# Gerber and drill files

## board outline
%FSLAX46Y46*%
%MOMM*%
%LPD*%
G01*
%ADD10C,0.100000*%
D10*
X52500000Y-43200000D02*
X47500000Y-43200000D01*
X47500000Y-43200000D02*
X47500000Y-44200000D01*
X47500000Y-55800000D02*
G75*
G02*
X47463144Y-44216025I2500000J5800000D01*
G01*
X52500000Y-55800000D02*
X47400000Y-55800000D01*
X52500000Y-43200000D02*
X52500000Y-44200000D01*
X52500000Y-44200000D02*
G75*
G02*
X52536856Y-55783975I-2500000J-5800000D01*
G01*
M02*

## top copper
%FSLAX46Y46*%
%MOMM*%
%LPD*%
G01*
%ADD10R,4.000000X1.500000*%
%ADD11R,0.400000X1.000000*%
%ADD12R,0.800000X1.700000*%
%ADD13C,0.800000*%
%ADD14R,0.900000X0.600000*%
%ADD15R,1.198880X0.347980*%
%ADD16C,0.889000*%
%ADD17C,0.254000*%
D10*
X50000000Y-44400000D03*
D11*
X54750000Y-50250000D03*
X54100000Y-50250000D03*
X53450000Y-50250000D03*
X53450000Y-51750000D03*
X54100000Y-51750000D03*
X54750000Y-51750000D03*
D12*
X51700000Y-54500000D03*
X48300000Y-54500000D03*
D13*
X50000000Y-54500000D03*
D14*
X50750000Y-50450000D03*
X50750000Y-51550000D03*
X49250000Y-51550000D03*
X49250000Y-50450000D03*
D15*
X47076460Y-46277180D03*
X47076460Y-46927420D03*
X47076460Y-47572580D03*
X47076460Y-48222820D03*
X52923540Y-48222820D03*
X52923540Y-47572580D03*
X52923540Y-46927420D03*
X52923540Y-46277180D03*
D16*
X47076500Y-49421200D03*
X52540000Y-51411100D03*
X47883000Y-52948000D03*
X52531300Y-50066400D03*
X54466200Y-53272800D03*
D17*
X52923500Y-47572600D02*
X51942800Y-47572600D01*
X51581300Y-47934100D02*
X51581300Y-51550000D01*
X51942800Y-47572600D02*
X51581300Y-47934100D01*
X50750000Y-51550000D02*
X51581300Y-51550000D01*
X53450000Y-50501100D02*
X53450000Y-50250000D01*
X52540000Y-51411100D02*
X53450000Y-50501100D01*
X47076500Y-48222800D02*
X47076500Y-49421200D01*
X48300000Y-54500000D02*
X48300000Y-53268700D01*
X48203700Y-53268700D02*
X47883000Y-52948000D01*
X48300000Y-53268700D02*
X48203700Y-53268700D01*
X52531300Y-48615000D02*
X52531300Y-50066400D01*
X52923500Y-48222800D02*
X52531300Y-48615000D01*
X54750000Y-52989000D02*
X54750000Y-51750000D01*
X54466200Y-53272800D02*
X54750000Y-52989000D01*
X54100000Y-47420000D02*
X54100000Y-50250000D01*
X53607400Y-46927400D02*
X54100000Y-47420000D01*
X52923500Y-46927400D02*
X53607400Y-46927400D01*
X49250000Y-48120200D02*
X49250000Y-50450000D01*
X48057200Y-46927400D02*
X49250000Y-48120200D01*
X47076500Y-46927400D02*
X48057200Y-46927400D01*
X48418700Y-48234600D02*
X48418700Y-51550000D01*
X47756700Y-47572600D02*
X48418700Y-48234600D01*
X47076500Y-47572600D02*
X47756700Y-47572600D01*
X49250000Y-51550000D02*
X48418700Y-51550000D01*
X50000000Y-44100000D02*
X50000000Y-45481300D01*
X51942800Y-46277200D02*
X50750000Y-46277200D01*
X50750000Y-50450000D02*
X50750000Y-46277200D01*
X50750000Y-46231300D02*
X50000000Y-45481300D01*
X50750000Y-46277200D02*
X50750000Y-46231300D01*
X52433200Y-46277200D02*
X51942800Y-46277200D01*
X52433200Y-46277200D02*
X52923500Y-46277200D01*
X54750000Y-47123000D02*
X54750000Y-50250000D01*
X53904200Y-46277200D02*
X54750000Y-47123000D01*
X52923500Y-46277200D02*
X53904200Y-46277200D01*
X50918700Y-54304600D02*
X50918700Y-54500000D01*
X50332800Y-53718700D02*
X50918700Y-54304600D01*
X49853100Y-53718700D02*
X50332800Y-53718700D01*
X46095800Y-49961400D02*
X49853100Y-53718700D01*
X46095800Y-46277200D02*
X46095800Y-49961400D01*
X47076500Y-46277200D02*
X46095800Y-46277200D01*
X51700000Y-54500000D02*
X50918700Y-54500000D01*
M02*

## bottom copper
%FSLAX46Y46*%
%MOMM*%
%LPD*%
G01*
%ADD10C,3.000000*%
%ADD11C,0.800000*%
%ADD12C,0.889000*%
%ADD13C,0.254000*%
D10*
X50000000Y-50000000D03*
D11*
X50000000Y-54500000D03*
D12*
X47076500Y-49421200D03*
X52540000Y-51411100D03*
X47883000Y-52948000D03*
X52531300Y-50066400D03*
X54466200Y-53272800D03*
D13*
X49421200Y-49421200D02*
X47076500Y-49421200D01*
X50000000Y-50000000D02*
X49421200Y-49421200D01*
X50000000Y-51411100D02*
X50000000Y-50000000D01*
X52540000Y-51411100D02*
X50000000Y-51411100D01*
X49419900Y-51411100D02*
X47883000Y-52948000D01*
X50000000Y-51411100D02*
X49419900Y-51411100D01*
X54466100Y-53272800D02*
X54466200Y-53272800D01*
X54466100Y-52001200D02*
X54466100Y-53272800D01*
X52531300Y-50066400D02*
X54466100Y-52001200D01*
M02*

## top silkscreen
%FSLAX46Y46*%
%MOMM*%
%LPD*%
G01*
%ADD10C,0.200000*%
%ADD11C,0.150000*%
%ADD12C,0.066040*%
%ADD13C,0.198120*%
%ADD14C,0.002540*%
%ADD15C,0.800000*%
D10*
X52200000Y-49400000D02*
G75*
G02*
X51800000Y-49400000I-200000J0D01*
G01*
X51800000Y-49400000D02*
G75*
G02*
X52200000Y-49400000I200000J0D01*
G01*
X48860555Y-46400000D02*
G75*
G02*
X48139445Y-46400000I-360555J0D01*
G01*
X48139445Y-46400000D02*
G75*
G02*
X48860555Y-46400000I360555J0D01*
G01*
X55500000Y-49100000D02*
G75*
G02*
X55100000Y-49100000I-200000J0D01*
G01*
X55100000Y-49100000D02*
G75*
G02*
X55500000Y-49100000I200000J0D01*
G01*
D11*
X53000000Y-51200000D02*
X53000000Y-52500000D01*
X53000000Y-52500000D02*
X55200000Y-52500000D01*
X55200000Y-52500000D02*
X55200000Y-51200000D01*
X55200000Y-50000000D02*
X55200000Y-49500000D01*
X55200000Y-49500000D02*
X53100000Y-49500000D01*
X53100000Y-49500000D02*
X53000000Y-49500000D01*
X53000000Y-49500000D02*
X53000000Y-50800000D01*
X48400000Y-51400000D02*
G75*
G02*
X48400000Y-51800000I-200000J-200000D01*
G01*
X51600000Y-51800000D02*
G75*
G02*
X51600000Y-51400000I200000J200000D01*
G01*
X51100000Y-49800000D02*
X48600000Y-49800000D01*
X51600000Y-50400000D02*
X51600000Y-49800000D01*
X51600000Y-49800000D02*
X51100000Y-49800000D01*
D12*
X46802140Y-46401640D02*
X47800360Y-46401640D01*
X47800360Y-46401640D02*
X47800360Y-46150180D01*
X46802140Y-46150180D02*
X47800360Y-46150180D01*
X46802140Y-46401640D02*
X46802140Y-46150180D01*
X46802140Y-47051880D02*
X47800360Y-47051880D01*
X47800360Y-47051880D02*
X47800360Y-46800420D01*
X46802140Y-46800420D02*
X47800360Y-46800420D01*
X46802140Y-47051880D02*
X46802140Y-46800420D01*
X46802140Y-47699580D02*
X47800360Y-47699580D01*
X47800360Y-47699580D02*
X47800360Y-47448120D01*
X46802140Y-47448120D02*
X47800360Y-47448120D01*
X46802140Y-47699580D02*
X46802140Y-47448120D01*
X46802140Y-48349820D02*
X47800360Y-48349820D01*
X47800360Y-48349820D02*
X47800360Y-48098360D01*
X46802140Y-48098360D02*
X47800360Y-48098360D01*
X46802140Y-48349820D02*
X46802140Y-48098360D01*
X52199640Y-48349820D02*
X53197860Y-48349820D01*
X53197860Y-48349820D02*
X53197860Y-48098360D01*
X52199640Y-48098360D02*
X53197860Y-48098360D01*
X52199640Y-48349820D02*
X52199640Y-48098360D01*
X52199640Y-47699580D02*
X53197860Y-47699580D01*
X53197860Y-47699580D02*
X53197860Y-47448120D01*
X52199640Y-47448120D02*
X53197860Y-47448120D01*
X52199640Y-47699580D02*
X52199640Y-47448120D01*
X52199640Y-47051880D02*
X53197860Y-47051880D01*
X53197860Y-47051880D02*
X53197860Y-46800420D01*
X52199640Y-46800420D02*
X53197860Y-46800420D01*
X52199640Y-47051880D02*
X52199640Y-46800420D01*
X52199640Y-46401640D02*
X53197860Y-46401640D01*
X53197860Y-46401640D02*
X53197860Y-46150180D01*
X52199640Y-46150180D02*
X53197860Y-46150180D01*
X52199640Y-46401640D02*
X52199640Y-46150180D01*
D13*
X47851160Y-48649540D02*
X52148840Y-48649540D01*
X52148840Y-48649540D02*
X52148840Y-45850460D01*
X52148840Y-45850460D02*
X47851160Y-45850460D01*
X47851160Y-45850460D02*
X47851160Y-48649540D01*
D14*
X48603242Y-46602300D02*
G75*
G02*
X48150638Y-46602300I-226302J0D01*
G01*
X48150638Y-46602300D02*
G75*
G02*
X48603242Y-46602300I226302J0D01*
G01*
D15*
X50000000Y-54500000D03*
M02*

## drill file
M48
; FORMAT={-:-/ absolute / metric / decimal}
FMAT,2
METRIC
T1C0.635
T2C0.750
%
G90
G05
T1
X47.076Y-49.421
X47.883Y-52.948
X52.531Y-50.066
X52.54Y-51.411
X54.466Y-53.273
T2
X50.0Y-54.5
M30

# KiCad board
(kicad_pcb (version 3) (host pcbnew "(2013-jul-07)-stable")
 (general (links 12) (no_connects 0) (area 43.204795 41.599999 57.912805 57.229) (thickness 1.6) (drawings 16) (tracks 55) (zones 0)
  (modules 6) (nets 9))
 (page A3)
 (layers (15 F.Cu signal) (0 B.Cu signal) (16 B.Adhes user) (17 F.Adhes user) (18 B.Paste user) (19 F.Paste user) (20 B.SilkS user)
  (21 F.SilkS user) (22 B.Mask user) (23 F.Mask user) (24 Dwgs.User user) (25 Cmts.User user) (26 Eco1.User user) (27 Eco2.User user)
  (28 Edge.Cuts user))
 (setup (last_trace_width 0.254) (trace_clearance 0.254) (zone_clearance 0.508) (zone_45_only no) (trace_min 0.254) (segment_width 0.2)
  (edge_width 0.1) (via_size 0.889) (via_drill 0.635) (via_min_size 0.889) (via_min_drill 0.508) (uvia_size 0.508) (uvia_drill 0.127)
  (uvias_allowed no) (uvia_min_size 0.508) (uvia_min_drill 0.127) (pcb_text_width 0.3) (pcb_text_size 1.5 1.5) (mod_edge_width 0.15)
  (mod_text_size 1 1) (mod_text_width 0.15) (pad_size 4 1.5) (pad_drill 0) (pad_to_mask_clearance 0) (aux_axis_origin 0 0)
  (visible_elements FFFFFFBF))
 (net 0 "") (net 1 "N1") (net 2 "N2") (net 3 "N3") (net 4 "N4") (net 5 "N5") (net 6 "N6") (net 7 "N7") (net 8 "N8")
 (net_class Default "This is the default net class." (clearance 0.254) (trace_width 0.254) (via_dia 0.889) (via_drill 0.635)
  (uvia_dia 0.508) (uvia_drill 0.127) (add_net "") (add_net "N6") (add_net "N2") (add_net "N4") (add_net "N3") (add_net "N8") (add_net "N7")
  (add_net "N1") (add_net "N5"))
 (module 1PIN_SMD (layer F.Cu) (at 50 44.4)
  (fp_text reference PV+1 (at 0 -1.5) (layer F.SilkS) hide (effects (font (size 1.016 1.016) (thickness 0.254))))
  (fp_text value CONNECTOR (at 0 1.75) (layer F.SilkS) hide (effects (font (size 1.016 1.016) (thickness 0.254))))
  (pad 1 smd rect (at 0 0) (size 4 1.5) (layers F.Cu F.Paste F.Mask) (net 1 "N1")))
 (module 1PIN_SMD (layer B.Cu) (at 50 50)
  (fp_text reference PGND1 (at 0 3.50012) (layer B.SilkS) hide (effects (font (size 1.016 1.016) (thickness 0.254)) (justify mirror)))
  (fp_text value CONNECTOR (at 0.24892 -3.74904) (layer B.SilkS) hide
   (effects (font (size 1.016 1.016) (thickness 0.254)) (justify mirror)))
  (pad 1 smd circle (at 0 0) (size 3 3) (layers B.Cu B.Paste B.Mask) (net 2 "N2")))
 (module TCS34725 (layer F.Cu) (at 54.1 51 90)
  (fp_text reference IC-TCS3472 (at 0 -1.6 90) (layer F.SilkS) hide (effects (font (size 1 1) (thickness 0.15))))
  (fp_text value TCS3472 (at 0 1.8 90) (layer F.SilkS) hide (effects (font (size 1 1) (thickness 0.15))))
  (fp_line (start -0.2 -1.1) (end -1.5 -1.1) (layer F.SilkS) (width 0.15))
  (fp_line (start -1.5 -1.1) (end -1.5 1.1) (layer F.SilkS) (width 0.15))
  (fp_line (start -1.5 1.1) (end -0.2 1.1) (layer F.SilkS) (width 0.15))
  (fp_line (start 1 1.1) (end 1.5 1.1) (layer F.SilkS) (width 0.15))
  (fp_line (start 1.5 1.1) (end 1.5 -1) (layer F.SilkS) (width 0.15))
  (fp_line (start 1.5 -1) (end 1.5 -1.1) (layer F.SilkS) (width 0.15))
  (fp_line (start 1.5 -1.1) (end 0.2 -1.1) (layer F.SilkS) (width 0.15))
  (pad 1 smd rect (at 0.75 0.65 90) (size 1 0.4) (layers F.Cu F.Paste F.Mask) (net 1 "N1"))
  (pad 2 smd rect (at 0.75 0 90) (size 1 0.4) (layers F.Cu F.Paste F.Mask) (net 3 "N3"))
  (pad 3 smd rect (at 0.75 -0.65 90) (size 1 0.4) (layers F.Cu F.Paste F.Mask) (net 2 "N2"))
  (pad 4 smd rect (at -0.75 -0.65 90) (size 1 0.4) (layers F.Cu F.Paste F.Mask))
  (pad 5 smd rect (at -0.75 0 90) (size 1 0.4) (layers F.Cu F.Paste F.Mask))
  (pad 6 smd rect (at -0.75 0.65 90) (size 1 0.4) (layers F.Cu F.Paste F.Mask) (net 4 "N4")))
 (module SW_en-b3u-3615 (layer F.Cu) (at 50 54.5 180)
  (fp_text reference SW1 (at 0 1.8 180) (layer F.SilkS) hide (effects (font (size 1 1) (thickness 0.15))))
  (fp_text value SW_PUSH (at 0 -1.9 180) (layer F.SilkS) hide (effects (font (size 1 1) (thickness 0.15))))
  (pad 1 smd rect (at -1.7 0 180) (size 0.8 1.7) (layers F.Cu F.Paste F.Mask) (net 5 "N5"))
  (pad 2 smd rect (at 1.7 0 180) (size 0.8 1.7) (layers F.Cu F.Paste F.Mask) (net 2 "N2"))
  (pad "" thru_hole circle (at 0 0 180) (size 0.8 0.8) (drill 0.75) (layers *.Cu *.Mask F.SilkS)))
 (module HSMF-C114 (layer F.Cu) (at 50 51 180)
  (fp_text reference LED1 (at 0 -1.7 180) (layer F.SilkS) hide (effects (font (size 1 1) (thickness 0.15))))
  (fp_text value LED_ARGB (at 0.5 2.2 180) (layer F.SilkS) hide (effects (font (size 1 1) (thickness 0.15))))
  (fp_arc (start 1.8 -0.6) (end 1.6 -0.4) (angle 90) (layer F.SilkS) (width 0.15))
  (fp_arc (start -1.8 -0.6) (end -1.6 -0.8) (angle 90) (layer F.SilkS) (width 0.15))
  (fp_line (start -1.1 1.2) (end 1.4 1.2) (layer F.SilkS) (width 0.15))
  (fp_line (start -1.6 0.6) (end -1.6 1.2) (layer F.SilkS) (width 0.15))
  (fp_line (start -1.6 1.2) (end -1.1 1.2) (layer F.SilkS) (width 0.15))
  (pad 1 smd rect (at -0.75 0.55 180) (size 0.9 0.6) (layers F.Cu F.Paste F.Mask) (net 1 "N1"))
  (pad 2 smd rect (at -0.75 -0.55 180) (size 0.9 0.6) (layers F.Cu F.Paste F.Mask) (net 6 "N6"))
  (pad 3 smd rect (at 0.75 -0.55 180) (size 0.9 0.6) (layers F.Cu F.Paste F.Mask) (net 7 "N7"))
  (pad 4 smd rect (at 0.75 0.55 180) (size 0.9 0.6) (layers F.Cu F.Paste F.Mask) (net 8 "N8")))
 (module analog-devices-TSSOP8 (layer F.Cu) (at 50 47.25)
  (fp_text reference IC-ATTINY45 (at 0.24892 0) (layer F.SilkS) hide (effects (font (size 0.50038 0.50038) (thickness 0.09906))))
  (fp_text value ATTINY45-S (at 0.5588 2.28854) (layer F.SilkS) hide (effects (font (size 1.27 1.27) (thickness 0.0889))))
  (fp_line (start -3.19786 -0.84836) (end -2.19964 -0.84836) (layer F.SilkS) (width 0.06604))
  (fp_line (start -2.19964 -0.84836) (end -2.19964 -1.09982) (layer F.SilkS) (width 0.06604))
  (fp_line (start -3.19786 -1.09982) (end -2.19964 -1.09982) (layer F.SilkS) (width 0.06604))
  (fp_line (start -3.19786 -0.84836) (end -3.19786 -1.09982) (layer F.SilkS) (width 0.06604))
  (fp_line (start -3.19786 -0.19812) (end -2.19964 -0.19812) (layer F.SilkS) (width 0.06604))
  (fp_line (start -2.19964 -0.19812) (end -2.19964 -0.44958) (layer F.SilkS) (width 0.06604))
  (fp_line (start -3.19786 -0.44958) (end -2.19964 -0.44958) (layer F.SilkS) (width 0.06604))
  (fp_line (start -3.19786 -0.19812) (end -3.19786 -0.44958) (layer F.SilkS) (width 0.06604))
  (fp_line (start -3.19786 0.44958) (end -2.19964 0.44958) (layer F.SilkS) (width 0.06604))
  (fp_line (start -2.19964 0.44958) (end -2.19964 0.19812) (layer F.SilkS) (width 0.06604))
  (fp_line (start -3.19786 0.19812) (end -2.19964 0.19812) (layer F.SilkS) (width 0.06604))
  (fp_line (start -3.19786 0.44958) (end -3.19786 0.19812) (layer F.SilkS) (width 0.06604))
  (fp_line (start -3.19786 1.09982) (end -2.19964 1.09982) (layer F.SilkS) (width 0.06604))
  (fp_line (start -2.19964 1.09982) (end -2.19964 0.84836) (layer F.SilkS) (width 0.06604))
  (fp_line (start -3.19786 0.84836) (end -2.19964 0.84836) (layer F.SilkS) (width 0.06604))
  (fp_line (start -3.19786 1.09982) (end -3.19786 0.84836) (layer F.SilkS) (width 0.06604))
  (fp_line (start 2.19964 1.09982) (end 3.19786 1.09982) (layer F.SilkS) (width 0.06604))
  (fp_line (start 3.19786 1.09982) (end 3.19786 0.84836) (layer F.SilkS) (width 0.06604))
  (fp_line (start 2.19964 0.84836) (end 3.19786 0.84836) (layer F.SilkS) (width 0.06604))
  (fp_line (start 2.19964 1.09982) (end 2.19964 0.84836) (layer F.SilkS) (width 0.06604))
  (fp_line (start 2.19964 0.44958) (end 3.19786 0.44958) (layer F.SilkS) (width 0.06604))
  (fp_line (start 3.19786 0.44958) (end 3.19786 0.19812) (layer F.SilkS) (width 0.06604))
  (fp_line (start 2.19964 0.19812) (end 3.19786 0.19812) (layer F.SilkS) (width 0.06604))
  (fp_line (start 2.19964 0.44958) (end 2.19964 0.19812) (layer F.SilkS) (width 0.06604))
  (fp_line (start 2.19964 -0.19812) (end 3.19786 -0.19812) (layer F.SilkS) (width 0.06604))
  (fp_line (start 3.19786 -0.19812) (end 3.19786 -0.44958) (layer F.SilkS) (width 0.06604))
  (fp_line (start 2.19964 -0.44958) (end 3.19786 -0.44958) (layer F.SilkS) (width 0.06604))
  (fp_line (start 2.19964 -0.19812) (end 2.19964 -0.44958) (layer F.SilkS) (width 0.06604))
  (fp_line (start 2.19964 -0.84836) (end 3.19786 -0.84836) (layer F.SilkS) (width 0.06604))
  (fp_line (start 3.19786 -0.84836) (end 3.19786 -1.09982) (layer F.SilkS) (width 0.06604))
  (fp_line (start 2.19964 -1.09982) (end 3.19786 -1.09982) (layer F.SilkS) (width 0.06604))
  (fp_line (start 2.19964 -0.84836) (end 2.19964 -1.09982) (layer F.SilkS) (width 0.06604))
  (fp_line (start -2.14884 1.39954) (end 2.14884 1.39954) (layer F.SilkS) (width 0.19812))
  (fp_line (start 2.14884 1.39954) (end 2.14884 -1.39954) (layer F.SilkS) (width 0.19812))
  (fp_line (start 2.14884 -1.39954) (end -2.14884 -1.39954) (layer F.SilkS) (width 0.19812))
  (fp_line (start -2.14884 -1.39954) (end -2.14884 1.39954) (layer F.SilkS) (width 0.19812))
  (fp_circle (center -1.62306 -0.6477) (end -1.78308 -0.80772) (layer F.SilkS) (width 0.00254))
  (pad 1 smd rect (at -2.92354 -0.97282) (size 1.19888 0.34798) (layers F.Cu F.Paste F.Mask) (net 5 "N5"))
  (pad 2 smd rect (at -2.92354 -0.32258) (size 1.19888 0.34798) (layers F.Cu F.Paste F.Mask) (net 8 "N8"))
  (pad 3 smd rect (at -2.92354 0.32258) (size 1.19888 0.34798) (layers F.Cu F.Paste F.Mask) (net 7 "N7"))
  (pad 4 smd rect (at -2.92354 0.97282) (size 1.19888 0.34798) (layers F.Cu F.Paste F.Mask) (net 2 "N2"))
  (pad 5 smd rect (at 2.92354 0.97282) (size 1.19888 0.34798) (layers F.Cu F.Paste F.Mask) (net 4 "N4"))
  (pad 6 smd rect (at 2.92354 0.32258) (size 1.19888 0.34798) (layers F.Cu F.Paste F.Mask) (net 6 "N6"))
  (pad 7 smd rect (at 2.92354 -0.32258) (size 1.19888 0.34798) (layers F.Cu F.Paste F.Mask) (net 3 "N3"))
  (pad 8 smd rect (at 2.92354 -0.97282) (size 1.19888 0.34798) (layers F.Cu F.Paste F.Mask) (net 1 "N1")))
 (gr_line (start 52.5 43.2) (end 47.5 43.2) (angle 90) (layer Edge.Cuts) (width 0.1))
 (gr_line (start 47.5 43.2) (end 47.5 44.2) (angle 90) (layer Edge.Cuts) (width 0.1))
 (gr_arc (start 50 50) (end 47.5 55.8) (angle 133) (layer Edge.Cuts) (width 0.1))
 (gr_line (start 52.5 55.8) (end 47.4 55.8) (angle 90) (layer Edge.Cuts) (width 0.1))
 (gr_line (start 52.5 43.2) (end 52.5 44.2) (angle 90) (layer Edge.Cuts) (width 0.1))
 (gr_arc (start 50 50) (end 52.5 44.2) (angle 133) (layer Edge.Cuts) (width 0.1))
 (gr_circle (center 52 49.4) (end 52 49.2) (layer F.SilkS) (width 0.2))
 (gr_circle (center 48.5 46.4) (end 48.8 46.6) (layer F.SilkS) (width 0.2))
 (gr_circle (center 55.3 49.1) (end 55.3 48.9) (layer F.SilkS) (width 0.2))
 (segment (start 52.9235 47.5726) (end 51.9428 47.5726) (width 0.254) (layer F.Cu) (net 6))
 (segment (start 51.5813 47.9341) (end 51.5813 51.55) (width 0.254) (layer F.Cu) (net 6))
 (segment (start 51.9428 47.5726) (end 51.5813 47.9341) (width 0.254) (layer F.Cu) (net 6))
 (segment (start 50.75 51.55) (end 51.5813 51.55) (width 0.254) (layer F.Cu) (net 6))
 (via (at 47.0765 49.4212) (size 0.889) (layers F.Cu B.Cu) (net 2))
 (via (at 52.54 51.4111) (size 0.889) (layers F.Cu B.Cu) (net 2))
 (via (at 47.883 52.948) (size 0.889) (layers F.Cu B.Cu) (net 2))
 (segment (start 53.45 50.5011) (end 53.45 50.25) (width 0.254) (layer F.Cu) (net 2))
 (segment (start 52.54 51.4111) (end 53.45 50.5011) (width 0.254) (layer F.Cu) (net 2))
 (segment (start 49.4212 49.4212) (end 47.0765 49.4212) (width 0.254) (layer B.Cu) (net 2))
 (segment (start 50 50) (end 49.4212 49.4212) (width 0.254) (layer B.Cu) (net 2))
 (segment (start 47.0765 48.2228) (end 47.0765 49.4212) (width 0.254) (layer F.Cu) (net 2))
 (segment (start 48.3 54.5) (end 48.3 53.2687) (width 0.254) (layer F.Cu) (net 2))
 (segment (start 48.2037 53.2687) (end 47.883 52.948) (width 0.254) (layer F.Cu) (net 2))
 (segment (start 48.3 53.2687) (end 48.2037 53.2687) (width 0.254) (layer F.Cu) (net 2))
 (segment (start 50 51.4111) (end 50 50) (width 0.254) (layer B.Cu) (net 2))
 (segment (start 52.54 51.4111) (end 50 51.4111) (width 0.254) (layer B.Cu) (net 2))
 (segment (start 49.4199 51.4111) (end 47.883 52.948) (width 0.254) (layer B.Cu) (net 2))
 (segment (start 50 51.4111) (end 49.4199 51.4111) (width 0.254) (layer B.Cu) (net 2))
 (via (at 52.5313 50.0664) (size 0.889) (layers F.Cu B.Cu) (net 4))
 (via (at 54.4662 53.2728) (size 0.889) (layers F.Cu B.Cu) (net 4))
 (segment (start 52.5313 48.615) (end 52.5313 50.0664) (width 0.254) (layer F.Cu) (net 4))
 (segment (start 52.9235 48.2228) (end 52.5313 48.615) (width 0.254) (layer F.Cu) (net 4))
 (segment (start 54.4661 53.2728) (end 54.4662 53.2728) (width 0.254) (layer B.Cu) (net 4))
 (segment (start 54.4661 52.0012) (end 54.4661 53.2728) (width 0.254) (layer B.Cu) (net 4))
 (segment (start 52.5313 50.0664) (end 54.4661 52.0012) (width 0.254) (layer B.Cu) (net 4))
 (segment (start 54.75 52.989) (end 54.75 51.75) (width 0.254) (layer F.Cu) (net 4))
 (segment (start 54.4662 53.2728) (end 54.75 52.989) (width 0.254) (layer F.Cu) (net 4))
 (segment (start 54.1 47.42) (end 54.1 50.25) (width 0.254) (layer F.Cu) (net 3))
 (segment (start 53.6074 46.9274) (end 54.1 47.42) (width 0.254) (layer F.Cu) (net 3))
 (segment (start 52.9235 46.9274) (end 53.6074 46.9274) (width 0.254) (layer F.Cu) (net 3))
 (segment (start 49.25 48.1202) (end 49.25 50.45) (width 0.254) (layer F.Cu) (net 8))
 (segment (start 48.0572 46.9274) (end 49.25 48.1202) (width 0.254) (layer F.Cu) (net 8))
 (segment (start 47.0765 46.9274) (end 48.0572 46.9274) (width 0.254) (layer F.Cu) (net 8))
 (segment (start 48.4187 48.2346) (end 48.4187 51.55) (width 0.254) (layer F.Cu) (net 7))
 (segment (start 47.7567 47.5726) (end 48.4187 48.2346) (width 0.254) (layer F.Cu) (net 7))
 (segment (start 47.0765 47.5726) (end 47.7567 47.5726) (width 0.254) (layer F.Cu) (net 7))
 (segment (start 49.25 51.55) (end 48.4187 51.55) (width 0.254) (layer F.Cu) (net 7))
 (segment (start 50 44.1) (end 50 45.4813) (width 0.254) (layer F.Cu) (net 1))
 (segment (start 51.9428 46.2772) (end 50.75 46.2772) (width 0.254) (layer F.Cu) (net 1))
 (segment (start 50.75 50.45) (end 50.75 46.2772) (width 0.254) (layer F.Cu) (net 1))
 (segment (start 50.75 46.2313) (end 50 45.4813) (width 0.254) (layer F.Cu) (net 1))
 (segment (start 50.75 46.2772) (end 50.75 46.2313) (width 0.254) (layer F.Cu) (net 1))
 (segment (start 52.4332 46.2772) (end 51.9428 46.2772) (width 0.254) (layer F.Cu) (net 1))
 (segment (start 52.4332 46.2772) (end 52.9235 46.2772) (width 0.254) (layer F.Cu) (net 1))
 (segment (start 54.75 47.123) (end 54.75 50.25) (width 0.254) (layer F.Cu) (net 1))
 (segment (start 53.9042 46.2772) (end 54.75 47.123) (width 0.254) (layer F.Cu) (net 1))
 (segment (start 52.9235 46.2772) (end 53.9042 46.2772) (width 0.254) (layer F.Cu) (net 1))
 (segment (start 50.9187 54.3046) (end 50.9187 54.5) (width 0.254) (layer F.Cu) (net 5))
 (segment (start 50.3328 53.7187) (end 50.9187 54.3046) (width 0.254) (layer F.Cu) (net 5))
 (segment (start 49.8531 53.7187) (end 50.3328 53.7187) (width 0.254) (layer F.Cu) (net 5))
 (segment (start 46.0958 49.9614) (end 49.8531 53.7187) (width 0.254) (layer F.Cu) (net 5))
 (segment (start 46.0958 46.2772) (end 46.0958 49.9614) (width 0.254) (layer F.Cu) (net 5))
 (segment (start 47.0765 46.2772) (end 46.0958 46.2772) (width 0.254) (layer F.Cu) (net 5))
 (segment (start 51.7 54.5) (end 50.9187 54.5) (width 0.254) (layer F.Cu) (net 5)))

